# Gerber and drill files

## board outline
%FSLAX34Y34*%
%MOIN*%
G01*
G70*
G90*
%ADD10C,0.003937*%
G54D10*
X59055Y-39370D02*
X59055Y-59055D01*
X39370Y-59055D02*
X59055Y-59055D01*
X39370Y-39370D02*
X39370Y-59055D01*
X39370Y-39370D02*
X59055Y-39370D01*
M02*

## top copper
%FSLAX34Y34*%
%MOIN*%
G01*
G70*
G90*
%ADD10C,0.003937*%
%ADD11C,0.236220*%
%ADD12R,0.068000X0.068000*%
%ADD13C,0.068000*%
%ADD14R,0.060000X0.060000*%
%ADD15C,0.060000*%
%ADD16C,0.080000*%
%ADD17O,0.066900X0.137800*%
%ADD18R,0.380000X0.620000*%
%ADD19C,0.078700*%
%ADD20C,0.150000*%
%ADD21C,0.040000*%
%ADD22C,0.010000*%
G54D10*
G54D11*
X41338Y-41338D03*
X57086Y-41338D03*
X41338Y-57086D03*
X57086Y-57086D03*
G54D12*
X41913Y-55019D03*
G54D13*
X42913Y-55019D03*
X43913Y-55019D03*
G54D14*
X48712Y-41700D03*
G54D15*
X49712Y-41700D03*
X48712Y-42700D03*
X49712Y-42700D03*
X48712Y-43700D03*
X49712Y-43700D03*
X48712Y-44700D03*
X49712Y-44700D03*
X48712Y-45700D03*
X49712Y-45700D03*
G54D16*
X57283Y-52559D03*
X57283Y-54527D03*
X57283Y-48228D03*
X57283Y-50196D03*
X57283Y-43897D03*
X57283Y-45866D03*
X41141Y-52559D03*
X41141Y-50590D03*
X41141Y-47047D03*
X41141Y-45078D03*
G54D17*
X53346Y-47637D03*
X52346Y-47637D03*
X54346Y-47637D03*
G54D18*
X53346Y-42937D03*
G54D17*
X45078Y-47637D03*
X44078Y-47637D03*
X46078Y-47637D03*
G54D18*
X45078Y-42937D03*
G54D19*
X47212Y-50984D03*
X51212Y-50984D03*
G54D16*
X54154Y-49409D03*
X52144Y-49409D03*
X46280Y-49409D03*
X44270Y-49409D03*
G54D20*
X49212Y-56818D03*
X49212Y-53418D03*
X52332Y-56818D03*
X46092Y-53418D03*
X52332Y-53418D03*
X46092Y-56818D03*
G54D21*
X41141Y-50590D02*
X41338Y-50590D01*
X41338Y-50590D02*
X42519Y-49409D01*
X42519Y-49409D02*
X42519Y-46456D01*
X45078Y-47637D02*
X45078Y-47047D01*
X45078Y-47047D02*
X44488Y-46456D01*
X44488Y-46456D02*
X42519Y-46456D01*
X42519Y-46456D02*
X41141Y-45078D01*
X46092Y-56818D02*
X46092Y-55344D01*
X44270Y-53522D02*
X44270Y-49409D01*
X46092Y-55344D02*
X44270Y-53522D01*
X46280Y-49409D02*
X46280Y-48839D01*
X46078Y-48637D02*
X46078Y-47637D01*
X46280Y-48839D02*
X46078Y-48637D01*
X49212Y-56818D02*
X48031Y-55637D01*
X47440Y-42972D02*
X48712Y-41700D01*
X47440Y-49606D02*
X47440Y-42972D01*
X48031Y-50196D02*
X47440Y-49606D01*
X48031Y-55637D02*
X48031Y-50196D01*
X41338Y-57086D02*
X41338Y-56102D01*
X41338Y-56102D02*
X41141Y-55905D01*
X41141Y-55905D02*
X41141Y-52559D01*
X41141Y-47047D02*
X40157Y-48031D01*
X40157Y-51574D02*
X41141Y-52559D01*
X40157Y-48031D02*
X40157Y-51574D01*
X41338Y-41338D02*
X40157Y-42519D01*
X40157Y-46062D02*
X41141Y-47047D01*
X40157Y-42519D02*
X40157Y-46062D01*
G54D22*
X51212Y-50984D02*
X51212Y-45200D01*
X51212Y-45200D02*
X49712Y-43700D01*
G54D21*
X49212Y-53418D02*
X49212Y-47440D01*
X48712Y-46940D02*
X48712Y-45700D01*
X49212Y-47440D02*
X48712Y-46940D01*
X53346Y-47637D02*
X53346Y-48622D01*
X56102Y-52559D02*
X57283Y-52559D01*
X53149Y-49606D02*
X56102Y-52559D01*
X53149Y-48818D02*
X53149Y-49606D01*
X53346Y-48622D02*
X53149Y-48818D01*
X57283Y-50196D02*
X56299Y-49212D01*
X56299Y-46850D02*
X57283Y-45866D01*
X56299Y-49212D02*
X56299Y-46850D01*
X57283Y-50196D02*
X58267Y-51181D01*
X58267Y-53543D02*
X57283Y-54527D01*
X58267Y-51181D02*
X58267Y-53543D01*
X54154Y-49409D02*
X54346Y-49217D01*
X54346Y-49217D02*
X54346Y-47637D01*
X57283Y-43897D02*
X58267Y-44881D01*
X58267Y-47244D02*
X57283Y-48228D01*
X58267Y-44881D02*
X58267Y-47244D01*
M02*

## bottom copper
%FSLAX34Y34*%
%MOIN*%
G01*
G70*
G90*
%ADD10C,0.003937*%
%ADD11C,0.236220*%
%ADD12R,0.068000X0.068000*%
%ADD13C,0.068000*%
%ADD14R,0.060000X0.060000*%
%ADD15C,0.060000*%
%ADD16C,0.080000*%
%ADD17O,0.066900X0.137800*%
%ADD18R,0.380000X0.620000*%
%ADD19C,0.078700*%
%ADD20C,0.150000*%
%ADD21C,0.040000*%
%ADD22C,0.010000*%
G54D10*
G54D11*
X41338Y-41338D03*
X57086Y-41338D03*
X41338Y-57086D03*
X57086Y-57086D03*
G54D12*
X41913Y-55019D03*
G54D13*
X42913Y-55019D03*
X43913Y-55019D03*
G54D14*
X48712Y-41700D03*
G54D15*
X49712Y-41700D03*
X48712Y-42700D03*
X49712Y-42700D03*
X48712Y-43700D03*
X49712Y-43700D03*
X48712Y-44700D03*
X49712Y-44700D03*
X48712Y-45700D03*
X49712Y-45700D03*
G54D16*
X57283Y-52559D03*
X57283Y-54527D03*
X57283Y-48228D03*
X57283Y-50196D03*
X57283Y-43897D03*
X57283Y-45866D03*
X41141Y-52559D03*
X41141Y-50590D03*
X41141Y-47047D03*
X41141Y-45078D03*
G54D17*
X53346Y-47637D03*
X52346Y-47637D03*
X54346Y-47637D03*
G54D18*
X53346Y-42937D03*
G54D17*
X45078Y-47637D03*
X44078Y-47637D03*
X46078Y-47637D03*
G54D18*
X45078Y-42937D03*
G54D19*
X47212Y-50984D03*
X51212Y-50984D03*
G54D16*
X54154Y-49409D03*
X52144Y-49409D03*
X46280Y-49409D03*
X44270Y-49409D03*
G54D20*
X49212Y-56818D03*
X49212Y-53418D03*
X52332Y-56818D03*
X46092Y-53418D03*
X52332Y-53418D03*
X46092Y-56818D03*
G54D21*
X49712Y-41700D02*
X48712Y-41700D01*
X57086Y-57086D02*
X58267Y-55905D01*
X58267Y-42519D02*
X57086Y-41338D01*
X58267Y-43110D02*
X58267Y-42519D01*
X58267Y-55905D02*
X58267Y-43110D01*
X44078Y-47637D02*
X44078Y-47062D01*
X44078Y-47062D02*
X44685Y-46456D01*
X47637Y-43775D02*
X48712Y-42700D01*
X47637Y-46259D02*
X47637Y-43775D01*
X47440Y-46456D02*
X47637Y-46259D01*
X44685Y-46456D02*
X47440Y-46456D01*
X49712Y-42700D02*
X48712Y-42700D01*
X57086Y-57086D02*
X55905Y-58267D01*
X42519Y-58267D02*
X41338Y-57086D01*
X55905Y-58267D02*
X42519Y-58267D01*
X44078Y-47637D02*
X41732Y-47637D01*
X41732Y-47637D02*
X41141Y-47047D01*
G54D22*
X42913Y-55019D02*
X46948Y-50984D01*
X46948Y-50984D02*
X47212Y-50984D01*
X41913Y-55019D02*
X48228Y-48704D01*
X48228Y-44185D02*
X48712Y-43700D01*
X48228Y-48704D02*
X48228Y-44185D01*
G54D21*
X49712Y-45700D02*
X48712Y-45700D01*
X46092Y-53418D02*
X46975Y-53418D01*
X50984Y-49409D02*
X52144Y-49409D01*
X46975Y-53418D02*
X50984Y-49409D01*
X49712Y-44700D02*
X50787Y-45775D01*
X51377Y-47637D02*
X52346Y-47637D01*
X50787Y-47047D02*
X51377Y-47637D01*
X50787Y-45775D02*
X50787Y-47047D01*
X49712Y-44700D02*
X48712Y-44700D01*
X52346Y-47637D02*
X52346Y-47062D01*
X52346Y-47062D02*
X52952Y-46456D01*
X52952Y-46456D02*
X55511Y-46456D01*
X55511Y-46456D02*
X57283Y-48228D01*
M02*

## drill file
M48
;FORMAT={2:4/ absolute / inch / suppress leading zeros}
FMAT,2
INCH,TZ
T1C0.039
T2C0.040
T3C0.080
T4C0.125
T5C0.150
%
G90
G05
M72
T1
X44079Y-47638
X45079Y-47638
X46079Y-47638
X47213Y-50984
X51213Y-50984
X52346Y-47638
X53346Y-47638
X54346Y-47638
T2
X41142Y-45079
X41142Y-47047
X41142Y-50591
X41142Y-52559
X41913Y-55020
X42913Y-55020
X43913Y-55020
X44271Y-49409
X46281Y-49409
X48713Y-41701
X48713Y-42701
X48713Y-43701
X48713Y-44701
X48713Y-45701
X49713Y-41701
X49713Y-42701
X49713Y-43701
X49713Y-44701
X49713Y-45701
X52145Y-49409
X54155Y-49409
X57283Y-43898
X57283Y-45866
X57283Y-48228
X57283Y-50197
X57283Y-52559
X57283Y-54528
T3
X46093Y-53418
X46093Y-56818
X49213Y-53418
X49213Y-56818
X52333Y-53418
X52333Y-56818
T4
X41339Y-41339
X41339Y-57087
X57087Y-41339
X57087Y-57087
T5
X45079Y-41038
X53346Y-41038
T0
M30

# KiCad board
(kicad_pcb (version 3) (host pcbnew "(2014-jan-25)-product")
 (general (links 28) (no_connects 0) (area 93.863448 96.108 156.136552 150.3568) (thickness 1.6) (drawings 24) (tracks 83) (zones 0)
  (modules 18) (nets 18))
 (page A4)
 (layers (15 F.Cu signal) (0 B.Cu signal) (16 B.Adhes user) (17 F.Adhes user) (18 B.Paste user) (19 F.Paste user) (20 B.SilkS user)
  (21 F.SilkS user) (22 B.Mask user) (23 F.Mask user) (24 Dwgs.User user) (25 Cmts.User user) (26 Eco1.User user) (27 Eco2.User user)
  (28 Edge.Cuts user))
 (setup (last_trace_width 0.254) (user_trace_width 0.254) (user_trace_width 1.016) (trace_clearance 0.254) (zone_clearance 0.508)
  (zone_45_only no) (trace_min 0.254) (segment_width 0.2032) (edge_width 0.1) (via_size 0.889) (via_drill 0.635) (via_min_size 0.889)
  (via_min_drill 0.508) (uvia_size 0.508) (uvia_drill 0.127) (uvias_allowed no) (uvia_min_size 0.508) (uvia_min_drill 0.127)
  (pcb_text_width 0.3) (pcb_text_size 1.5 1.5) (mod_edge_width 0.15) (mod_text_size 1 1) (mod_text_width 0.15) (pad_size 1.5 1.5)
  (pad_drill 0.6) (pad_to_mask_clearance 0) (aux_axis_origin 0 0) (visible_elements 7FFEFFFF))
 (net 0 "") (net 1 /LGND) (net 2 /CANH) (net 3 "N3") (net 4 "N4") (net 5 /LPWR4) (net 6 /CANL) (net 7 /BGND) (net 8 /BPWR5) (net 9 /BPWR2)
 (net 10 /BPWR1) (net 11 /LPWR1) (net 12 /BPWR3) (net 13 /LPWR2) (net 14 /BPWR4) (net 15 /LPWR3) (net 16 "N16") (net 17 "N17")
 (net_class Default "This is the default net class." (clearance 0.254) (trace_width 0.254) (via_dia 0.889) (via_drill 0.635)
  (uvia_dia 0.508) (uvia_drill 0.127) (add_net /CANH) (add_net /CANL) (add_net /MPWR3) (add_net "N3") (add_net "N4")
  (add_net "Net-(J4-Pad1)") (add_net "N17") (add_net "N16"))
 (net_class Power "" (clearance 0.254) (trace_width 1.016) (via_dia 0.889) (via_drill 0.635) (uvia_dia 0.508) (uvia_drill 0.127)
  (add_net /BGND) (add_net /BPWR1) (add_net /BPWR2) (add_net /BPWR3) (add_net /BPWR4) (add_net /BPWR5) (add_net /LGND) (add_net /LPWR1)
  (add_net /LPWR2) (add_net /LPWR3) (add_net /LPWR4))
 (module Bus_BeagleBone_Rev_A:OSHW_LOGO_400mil (layer B.Cu) (at 138.75 110.5)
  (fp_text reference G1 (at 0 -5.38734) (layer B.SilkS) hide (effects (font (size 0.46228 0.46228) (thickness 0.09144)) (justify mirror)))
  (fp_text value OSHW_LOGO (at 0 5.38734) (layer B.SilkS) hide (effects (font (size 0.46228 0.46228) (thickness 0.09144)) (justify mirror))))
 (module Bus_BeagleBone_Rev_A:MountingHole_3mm (layer F.Cu) (at 105 105)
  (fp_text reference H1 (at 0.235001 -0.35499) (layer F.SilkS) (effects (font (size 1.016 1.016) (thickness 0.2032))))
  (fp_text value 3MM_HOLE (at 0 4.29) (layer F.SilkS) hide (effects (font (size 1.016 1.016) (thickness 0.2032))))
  (pad 1 thru_hole circle (at 0 0) (size 6 6) (drill 3.175) (layers *.Cu *.SilkS *.Mask) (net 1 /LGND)))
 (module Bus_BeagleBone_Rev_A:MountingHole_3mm (layer F.Cu) (at 145 105)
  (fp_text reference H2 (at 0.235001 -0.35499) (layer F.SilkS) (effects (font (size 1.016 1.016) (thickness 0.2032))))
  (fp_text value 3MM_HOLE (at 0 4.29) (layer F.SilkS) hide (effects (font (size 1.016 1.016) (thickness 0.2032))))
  (pad 1 thru_hole circle (at 0 0) (size 6 6) (drill 3.175) (layers *.Cu *.SilkS *.Mask) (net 1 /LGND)))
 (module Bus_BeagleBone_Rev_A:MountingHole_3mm (layer F.Cu) (at 105 145)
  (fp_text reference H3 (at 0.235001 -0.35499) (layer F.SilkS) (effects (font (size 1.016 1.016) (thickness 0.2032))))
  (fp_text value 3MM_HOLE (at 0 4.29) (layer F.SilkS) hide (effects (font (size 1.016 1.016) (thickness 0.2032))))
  (pad 1 thru_hole circle (at 0 0) (size 6 6) (drill 3.175) (layers *.Cu *.SilkS *.Mask) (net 1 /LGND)))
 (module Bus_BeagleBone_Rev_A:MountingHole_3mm (layer F.Cu) (at 145 145)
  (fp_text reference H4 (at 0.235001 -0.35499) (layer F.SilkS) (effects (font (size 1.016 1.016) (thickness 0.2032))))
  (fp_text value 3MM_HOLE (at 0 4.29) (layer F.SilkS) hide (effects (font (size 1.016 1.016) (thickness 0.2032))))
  (pad 1 thru_hole circle (at 0 0) (size 6 6) (drill 3.175) (layers *.Cu *.SilkS *.Mask) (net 1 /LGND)))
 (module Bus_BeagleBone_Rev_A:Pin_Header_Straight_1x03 (layer F.Cu) (at 109 139.75)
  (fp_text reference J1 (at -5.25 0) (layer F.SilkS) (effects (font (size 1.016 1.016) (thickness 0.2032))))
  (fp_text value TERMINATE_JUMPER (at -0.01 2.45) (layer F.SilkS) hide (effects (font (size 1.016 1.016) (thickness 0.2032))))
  (pad 1 thru_hole rect (at -2.54 0) (size 1.7272 1.7272) (drill 1.016) (layers *.Cu *.Mask F.SilkS) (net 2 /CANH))
  (pad 2 thru_hole circle (at 0 0) (size 1.7272 1.7272) (drill 1.016) (layers *.Cu *.Mask F.SilkS) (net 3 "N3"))
  (pad 3 thru_hole circle (at 2.54 0) (size 1.7272 1.7272) (drill 1.016) (layers *.Cu *.Mask F.SilkS) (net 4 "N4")))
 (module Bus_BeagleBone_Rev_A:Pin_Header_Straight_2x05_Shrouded (layer F.Cu) (at 125 111 270)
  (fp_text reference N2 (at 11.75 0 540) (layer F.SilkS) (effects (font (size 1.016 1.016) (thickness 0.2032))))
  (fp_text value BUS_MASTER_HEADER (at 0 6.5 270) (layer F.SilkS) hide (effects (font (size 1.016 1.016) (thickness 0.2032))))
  (pad 1 thru_hole rect (at -5.08 1.27 270) (size 1.524 1.524) (drill 1.016) (layers *.Cu *.Mask F.SilkS) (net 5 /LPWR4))
  (pad 2 thru_hole circle (at -5.08 -1.27 270) (size 1.524 1.524) (drill 1.016) (layers *.Cu *.Mask F.SilkS) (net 5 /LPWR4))
  (pad 3 thru_hole circle (at -2.54 1.27 270) (size 1.524 1.524) (drill 1.016) (layers *.Cu *.Mask F.SilkS) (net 1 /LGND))
  (pad 4 thru_hole circle (at -2.54 -1.27 270) (size 1.524 1.524) (drill 1.016) (layers *.Cu *.Mask F.SilkS) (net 1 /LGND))
  (pad 5 thru_hole circle (at 0 1.27 270) (size 1.524 1.524) (drill 1.016) (layers *.Cu *.Mask F.SilkS) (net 2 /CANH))
  (pad 6 thru_hole circle (at 0 -1.27 270) (size 1.524 1.524) (drill 1.016) (layers *.Cu *.Mask F.SilkS) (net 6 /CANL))
  (pad 7 thru_hole circle (at 2.54 1.27 270) (size 1.524 1.524) (drill 1.016) (layers *.Cu *.Mask F.SilkS) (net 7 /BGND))
  (pad 8 thru_hole circle (at 2.54 -1.27 270) (size 1.524 1.524) (drill 1.016) (layers *.Cu *.Mask F.SilkS) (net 7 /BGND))
  (pad 9 thru_hole circle (at 5.08 1.27 270) (size 1.524 1.524) (drill 1.016) (layers *.Cu *.Mask F.SilkS) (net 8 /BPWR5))
  (pad 10 thru_hole circle (at 5.08 -1.27 270) (size 1.524 1.524) (drill 1.016) (layers *.Cu *.Mask F.SilkS) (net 8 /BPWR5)))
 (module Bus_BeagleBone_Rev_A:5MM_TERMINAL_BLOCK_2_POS (layer F.Cu) (at 145.5 136 270)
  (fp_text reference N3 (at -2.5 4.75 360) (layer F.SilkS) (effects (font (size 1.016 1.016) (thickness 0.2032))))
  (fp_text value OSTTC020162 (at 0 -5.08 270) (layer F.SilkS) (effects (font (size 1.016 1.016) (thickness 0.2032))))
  (pad 1 thru_hole circle (at -2.5 0 270) (size 2.032 2.032) (drill 1.016) (layers *.Cu *.Mask) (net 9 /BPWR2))
  (pad 2 thru_hole circle (at 2.5 0 270) (size 2.032 2.032) (drill 1.016) (layers *.Cu *.Mask) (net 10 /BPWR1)))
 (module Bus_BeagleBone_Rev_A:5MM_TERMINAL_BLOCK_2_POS (layer F.Cu) (at 145.5 125 270)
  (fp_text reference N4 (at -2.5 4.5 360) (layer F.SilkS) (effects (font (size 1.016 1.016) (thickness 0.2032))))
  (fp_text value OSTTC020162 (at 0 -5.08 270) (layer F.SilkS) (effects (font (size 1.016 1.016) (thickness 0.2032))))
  (pad 1 thru_hole circle (at -2.5 0 270) (size 2.032 2.032) (drill 1.016) (layers *.Cu *.Mask) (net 7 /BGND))
  (pad 2 thru_hole circle (at 2.5 0 270) (size 2.032 2.032) (drill 1.016) (layers *.Cu *.Mask) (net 10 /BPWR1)))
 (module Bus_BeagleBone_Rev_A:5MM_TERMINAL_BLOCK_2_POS (layer F.Cu) (at 145.5 114 270)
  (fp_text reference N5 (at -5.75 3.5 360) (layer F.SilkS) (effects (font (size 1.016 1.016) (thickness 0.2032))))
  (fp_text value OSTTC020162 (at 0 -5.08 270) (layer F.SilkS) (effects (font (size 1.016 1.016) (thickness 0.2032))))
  (pad 1 thru_hole circle (at -2.5 0 270) (size 2.032 2.032) (drill 1.016) (layers *.Cu *.Mask) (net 7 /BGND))
  (pad 2 thru_hole circle (at 2.5 0 270) (size 2.032 2.032) (drill 1.016) (layers *.Cu *.Mask) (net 10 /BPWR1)))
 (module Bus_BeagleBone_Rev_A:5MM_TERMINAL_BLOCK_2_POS (layer F.Cu) (at 104.5 131 90)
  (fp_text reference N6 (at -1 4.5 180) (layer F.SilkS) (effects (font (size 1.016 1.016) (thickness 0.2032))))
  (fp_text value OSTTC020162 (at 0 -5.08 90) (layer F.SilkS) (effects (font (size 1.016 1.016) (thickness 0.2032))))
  (pad 1 thru_hole circle (at -2.5 0 90) (size 2.032 2.032) (drill 1.016) (layers *.Cu *.Mask) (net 1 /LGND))
  (pad 2 thru_hole circle (at 2.5 0 90) (size 2.032 2.032) (drill 1.016) (layers *.Cu *.Mask) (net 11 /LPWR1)))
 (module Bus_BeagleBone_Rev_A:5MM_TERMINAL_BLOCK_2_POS (layer F.Cu) (at 104.5 117 90)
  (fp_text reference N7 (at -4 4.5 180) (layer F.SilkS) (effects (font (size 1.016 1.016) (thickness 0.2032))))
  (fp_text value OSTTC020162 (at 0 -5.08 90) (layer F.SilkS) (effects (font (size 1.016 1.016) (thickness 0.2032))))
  (pad 1 thru_hole circle (at -2.5 0 90) (size 2.032 2.032) (drill 1.016) (layers *.Cu *.Mask) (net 1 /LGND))
  (pad 2 thru_hole circle (at 2.5 0 90) (size 2.032 2.032) (drill 1.016) (layers *.Cu *.Mask) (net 11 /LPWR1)))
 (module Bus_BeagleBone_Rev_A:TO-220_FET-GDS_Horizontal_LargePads (layer F.Cu) (at 135.5 121)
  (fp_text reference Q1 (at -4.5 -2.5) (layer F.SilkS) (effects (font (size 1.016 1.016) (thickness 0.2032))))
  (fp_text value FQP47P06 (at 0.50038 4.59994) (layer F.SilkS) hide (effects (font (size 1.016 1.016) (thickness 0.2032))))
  (pad D thru_hole oval (at 0 0 90) (size 3.50012 1.69926) (drill 1.00076) (layers *.Cu *.Mask F.SilkS) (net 9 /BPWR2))
  (pad G thru_hole oval (at -2.54 0 90) (size 3.50012 1.69926) (drill 1.00076) (layers *.Cu *.Mask F.SilkS) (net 7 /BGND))
  (pad S thru_hole oval (at 2.54 0 90) (size 3.50012 1.69926) (drill 1.00076) (layers *.Cu *.Mask F.SilkS) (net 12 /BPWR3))
  (pad "" thru_hole rect (at 0 -16.764 90) (size 15.748 9.652) (drill 3.79984 (offset -4.826 0)) (layers *.Cu F.SilkS F.Mask)))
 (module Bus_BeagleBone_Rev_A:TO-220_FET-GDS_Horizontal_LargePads (layer F.Cu) (at 114.5 121)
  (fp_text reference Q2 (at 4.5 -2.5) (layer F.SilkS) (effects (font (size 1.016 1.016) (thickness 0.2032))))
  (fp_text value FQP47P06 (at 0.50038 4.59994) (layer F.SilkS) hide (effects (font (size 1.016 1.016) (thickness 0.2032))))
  (pad D thru_hole oval (at 0 0 90) (size 3.50012 1.69926) (drill 1.00076) (layers *.Cu *.Mask F.SilkS) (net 11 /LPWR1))
  (pad G thru_hole oval (at -2.54 0 90) (size 3.50012 1.69926) (drill 1.00076) (layers *.Cu *.Mask F.SilkS) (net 1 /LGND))
  (pad S thru_hole oval (at 2.54 0 90) (size 3.50012 1.69926) (drill 1.00076) (layers *.Cu *.Mask F.SilkS) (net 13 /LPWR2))
  (pad "" thru_hole rect (at 0 -16.764 90) (size 15.748 9.652) (drill 3.79984 (offset -4.826 0)) (layers *.Cu F.SilkS F.Mask)))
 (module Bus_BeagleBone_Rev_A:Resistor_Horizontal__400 (layer F.Cu) (at 125 129.5)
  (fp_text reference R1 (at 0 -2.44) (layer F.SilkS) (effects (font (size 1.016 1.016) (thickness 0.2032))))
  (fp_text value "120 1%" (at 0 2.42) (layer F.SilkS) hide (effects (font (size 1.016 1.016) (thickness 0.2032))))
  (pad 1 thru_hole circle (at -5.08 0) (size 1.99898 1.99898) (drill 1.00076) (layers *.Cu *.SilkS *.Mask) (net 3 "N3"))
  (pad 2 thru_hole circle (at 5.08 0) (size 1.99898 1.99898) (drill 1.00076) (layers *.Cu *.SilkS *.Mask) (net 6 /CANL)))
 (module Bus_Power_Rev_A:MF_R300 (layer F.Cu) (at 135 125.5 180)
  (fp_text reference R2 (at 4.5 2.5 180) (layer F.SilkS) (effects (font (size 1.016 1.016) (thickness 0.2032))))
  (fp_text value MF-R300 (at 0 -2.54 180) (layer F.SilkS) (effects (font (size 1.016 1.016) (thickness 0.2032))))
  (pad 1 thru_hole circle (at -2.5527 0 180) (size 2.032 2.032) (drill 1.016) (layers *.Cu *.Mask) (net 12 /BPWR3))
  (pad 2 thru_hole circle (at 2.5527 0 180) (size 2.032 2.032) (drill 1.016) (layers *.Cu *.Mask) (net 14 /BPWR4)))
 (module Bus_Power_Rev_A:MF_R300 (layer F.Cu) (at 115 125.5 180)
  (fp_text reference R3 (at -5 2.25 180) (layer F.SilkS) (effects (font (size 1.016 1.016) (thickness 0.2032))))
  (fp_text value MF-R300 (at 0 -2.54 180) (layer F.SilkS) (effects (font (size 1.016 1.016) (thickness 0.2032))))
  (pad 1 thru_hole circle (at -2.5527 0 180) (size 2.032 2.032) (drill 1.016) (layers *.Cu *.Mask) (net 13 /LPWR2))
  (pad 2 thru_hole circle (at 2.5527 0 180) (size 2.032 2.032) (drill 1.016) (layers *.Cu *.Mask) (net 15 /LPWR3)))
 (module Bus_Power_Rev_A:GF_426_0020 (layer F.Cu) (at 125 140)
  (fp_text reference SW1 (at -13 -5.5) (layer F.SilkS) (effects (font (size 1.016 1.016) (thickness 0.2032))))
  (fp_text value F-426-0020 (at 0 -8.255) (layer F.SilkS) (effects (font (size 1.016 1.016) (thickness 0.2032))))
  (pad 5 thru_hole circle (at 0 4.318) (size 3.81 3.81) (drill 2.032) (layers *.Cu *.Mask) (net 5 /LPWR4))
  (pad 2 thru_hole circle (at 0 -4.318) (size 3.81 3.81) (drill 2.032) (layers *.Cu *.Mask) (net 8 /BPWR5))
  (pad 6 thru_hole circle (at 7.9248 4.318) (size 3.81 3.81) (drill 2.032) (layers *.Cu *.Mask) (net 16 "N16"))
  (pad 1 thru_hole circle (at -7.9248 -4.318) (size 3.81 3.81) (drill 2.032) (layers *.Cu *.Mask) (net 14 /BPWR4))
  (pad 3 thru_hole circle (at 7.9248 -4.318) (size 3.81 3.81) (drill 2.032) (layers *.Cu *.Mask) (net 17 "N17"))
  (pad 4 thru_hole circle (at -7.9248 4.318) (size 3.81 3.81) (drill 2.032) (layers *.Cu *.Mask) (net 15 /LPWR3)))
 (gr_line (start 150 100) (end 150 150) (angle 90) (layer Edge.Cuts) (width 0.1))
 (gr_line (start 100 150) (end 150 150) (angle 90) (layer Edge.Cuts) (width 0.1))
 (gr_line (start 100 100) (end 100 150) (angle 90) (layer Edge.Cuts) (width 0.1))
 (gr_line (start 100 100) (end 150 100) (angle 90) (layer Edge.Cuts) (width 0.1))
 (segment (start 104.5 128.5) (end 105 128.5) (width 1.016) (layer F.Cu) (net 11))
 (segment (start 105 128.5) (end 108 125.5) (width 1.016) (layer F.Cu) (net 11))
 (segment (start 108 125.5) (end 108 118) (width 1.016) (layer F.Cu) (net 11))
 (segment (start 114.5 121) (end 114.5 119.5) (width 1.016) (layer F.Cu) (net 11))
 (segment (start 114.5 119.5) (end 113 118) (width 1.016) (layer F.Cu) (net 11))
 (segment (start 113 118) (end 108 118) (width 1.016) (layer F.Cu) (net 11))
 (segment (start 108 118) (end 104.5 114.5) (width 1.016) (layer F.Cu) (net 11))
 (segment (start 117.0752 144.318) (end 117.0752 140.5752) (width 1.016) (layer F.Cu) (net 15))
 (segment (start 112.4473 135.9473) (end 112.4473 125.5) (width 1.016) (layer F.Cu) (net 15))
 (segment (start 117.0752 140.5752) (end 112.4473 135.9473) (width 1.016) (layer F.Cu) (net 15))
 (segment (start 117.5527 125.5) (end 117.5527 124.0527) (width 1.016) (layer F.Cu) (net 13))
 (segment (start 117.04 123.54) (end 117.04 121) (width 1.016) (layer F.Cu) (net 13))
 (segment (start 117.5527 124.0527) (end 117.04 123.54) (width 1.016) (layer F.Cu) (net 13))
 (segment (start 125 144.318) (end 122 141.318) (width 1.016) (layer F.Cu) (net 5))
 (segment (start 120.5 109.15) (end 123.73 105.92) (width 1.016) (layer F.Cu) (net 5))
 (segment (start 120.5 126) (end 120.5 109.15) (width 1.016) (layer F.Cu) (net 5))
 (segment (start 122 127.5) (end 120.5 126) (width 1.016) (layer F.Cu) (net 5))
 (segment (start 122 141.318) (end 122 127.5) (width 1.016) (layer F.Cu) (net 5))
 (segment (start 126.27 105.92) (end 123.73 105.92) (width 1.016) (layer B.Cu) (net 5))
 (segment (start 145 145) (end 148 142) (width 1.016) (layer B.Cu) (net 1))
 (segment (start 148 108) (end 145 105) (width 1.016) (layer B.Cu) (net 1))
 (segment (start 148 109.5) (end 148 108) (width 1.016) (layer B.Cu) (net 1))
 (segment (start 148 142) (end 148 109.5) (width 1.016) (layer B.Cu) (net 1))
 (segment (start 111.96 121) (end 111.96 119.54) (width 1.016) (layer B.Cu) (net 1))
 (segment (start 111.96 119.54) (end 113.5 118) (width 1.016) (layer B.Cu) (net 1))
 (segment (start 121 111.19) (end 123.73 108.46) (width 1.016) (layer B.Cu) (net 1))
 (segment (start 121 117.5) (end 121 111.19) (width 1.016) (layer B.Cu) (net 1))
 (segment (start 120.5 118) (end 121 117.5) (width 1.016) (layer B.Cu) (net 1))
 (segment (start 113.5 118) (end 120.5 118) (width 1.016) (layer B.Cu) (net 1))
 (segment (start 126.27 108.46) (end 123.73 108.46) (width 1.016) (layer B.Cu) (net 1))
 (segment (start 145 145) (end 142 148) (width 1.016) (layer B.Cu) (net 1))
 (segment (start 108 148) (end 105 145) (width 1.016) (layer B.Cu) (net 1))
 (segment (start 142 148) (end 108 148) (width 1.016) (layer B.Cu) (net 1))
 (segment (start 105 145) (end 105 142.5) (width 1.016) (layer F.Cu) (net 1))
 (segment (start 105 142.5) (end 104.5 142) (width 1.016) (layer F.Cu) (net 1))
 (segment (start 104.5 142) (end 104.5 133.5) (width 1.016) (layer F.Cu) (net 1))
 (segment (start 104.5 119.5) (end 102 122) (width 1.016) (layer F.Cu) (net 1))
 (segment (start 102 131) (end 104.5 133.5) (width 1.016) (layer F.Cu) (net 1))
 (segment (start 102 122) (end 102 131) (width 1.016) (layer F.Cu) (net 1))
 (segment (start 111.96 121) (end 106 121) (width 1.016) (layer B.Cu) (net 1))
 (segment (start 106 121) (end 104.5 119.5) (width 1.016) (layer B.Cu) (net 1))
 (segment (start 105 105) (end 102 108) (width 1.016) (layer F.Cu) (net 1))
 (segment (start 102 117) (end 104.5 119.5) (width 1.016) (layer F.Cu) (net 1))
 (segment (start 102 108) (end 102 117) (width 1.016) (layer F.Cu) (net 1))
 (segment (start 109 139.75) (end 119.25 129.5) (width 0.254) (layer B.Cu) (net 3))
 (segment (start 119.25 129.5) (end 119.92 129.5) (width 0.254) (layer B.Cu) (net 3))
 (segment (start 106.46 139.75) (end 122.5 123.71) (width 0.254) (layer B.Cu) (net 2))
 (segment (start 122.5 112.23) (end 123.73 111) (width 0.254) (layer B.Cu) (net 2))
 (segment (start 122.5 123.71) (end 122.5 112.23) (width 0.254) (layer B.Cu) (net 2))
 (segment (start 130.08 129.5) (end 130.08 114.81) (width 0.254) (layer F.Cu) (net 6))
 (segment (start 130.08 114.81) (end 126.27 111) (width 0.254) (layer F.Cu) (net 6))
 (segment (start 125 135.682) (end 125 120.5) (width 1.016) (layer F.Cu) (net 8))
 (segment (start 123.73 119.23) (end 123.73 116.08) (width 1.016) (layer F.Cu) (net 8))
 (segment (start 125 120.5) (end 123.73 119.23) (width 1.016) (layer F.Cu) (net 8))
 (segment (start 126.27 116.08) (end 123.73 116.08) (width 1.016) (layer B.Cu) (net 8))
 (segment (start 135.5 121) (end 135.5 123.5) (width 1.016) (layer F.Cu) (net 9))
 (segment (start 142.5 133.5) (end 145.5 133.5) (width 1.016) (layer F.Cu) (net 9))
 (segment (start 135 126) (end 142.5 133.5) (width 1.016) (layer F.Cu) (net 9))
 (segment (start 135 124) (end 135 126) (width 1.016) (layer F.Cu) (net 9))
 (segment (start 135.5 123.5) (end 135 124) (width 1.016) (layer F.Cu) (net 9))
 (segment (start 145.5 127.5) (end 143 125) (width 1.016) (layer F.Cu) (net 10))
 (segment (start 143 119) (end 145.5 116.5) (width 1.016) (layer F.Cu) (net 10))
 (segment (start 143 125) (end 143 119) (width 1.016) (layer F.Cu) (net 10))
 (segment (start 145.5 127.5) (end 148 130) (width 1.016) (layer F.Cu) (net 10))
 (segment (start 148 136) (end 145.5 138.5) (width 1.016) (layer F.Cu) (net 10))
 (segment (start 148 130) (end 148 136) (width 1.016) (layer F.Cu) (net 10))
 (segment (start 137.5527 125.5) (end 138.04 125.0127) (width 1.016) (layer F.Cu) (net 12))
 (segment (start 138.04 125.0127) (end 138.04 121) (width 1.016) (layer F.Cu) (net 12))
 (segment (start 117.0752 135.682) (end 119.318 135.682) (width 1.016) (layer B.Cu) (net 14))
 (segment (start 129.5 125.5) (end 132.4473 125.5) (width 1.016) (layer B.Cu) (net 14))
 (segment (start 119.318 135.682) (end 129.5 125.5) (width 1.016) (layer B.Cu) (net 14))
 (segment (start 126.27 113.54) (end 129 116.27) (width 1.016) (layer B.Cu) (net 7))
 (segment (start 130.5 121) (end 132.96 121) (width 1.016) (layer B.Cu) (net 7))
 (segment (start 129 119.5) (end 130.5 121) (width 1.016) (layer B.Cu) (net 7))
 (segment (start 129 116.27) (end 129 119.5) (width 1.016) (layer B.Cu) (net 7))
 (segment (start 126.27 113.54) (end 123.73 113.54) (width 1.016) (layer B.Cu) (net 7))
 (segment (start 132.96 121) (end 132.96 119.54) (width 1.016) (layer B.Cu) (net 7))
 (segment (start 132.96 119.54) (end 134.5 118) (width 1.016) (layer B.Cu) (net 7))
 (segment (start 134.5 118) (end 141 118) (width 1.016) (layer B.Cu) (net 7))
 (segment (start 141 118) (end 145.5 122.5) (width 1.016) (layer B.Cu) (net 7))
 (segment (start 145.5 111.5) (end 148 114) (width 1.016) (layer F.Cu) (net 7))
 (segment (start 148 120) (end 145.5 122.5) (width 1.016) (layer F.Cu) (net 7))
 (segment (start 148 114) (end 148 120) (width 1.016) (layer F.Cu) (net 7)))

